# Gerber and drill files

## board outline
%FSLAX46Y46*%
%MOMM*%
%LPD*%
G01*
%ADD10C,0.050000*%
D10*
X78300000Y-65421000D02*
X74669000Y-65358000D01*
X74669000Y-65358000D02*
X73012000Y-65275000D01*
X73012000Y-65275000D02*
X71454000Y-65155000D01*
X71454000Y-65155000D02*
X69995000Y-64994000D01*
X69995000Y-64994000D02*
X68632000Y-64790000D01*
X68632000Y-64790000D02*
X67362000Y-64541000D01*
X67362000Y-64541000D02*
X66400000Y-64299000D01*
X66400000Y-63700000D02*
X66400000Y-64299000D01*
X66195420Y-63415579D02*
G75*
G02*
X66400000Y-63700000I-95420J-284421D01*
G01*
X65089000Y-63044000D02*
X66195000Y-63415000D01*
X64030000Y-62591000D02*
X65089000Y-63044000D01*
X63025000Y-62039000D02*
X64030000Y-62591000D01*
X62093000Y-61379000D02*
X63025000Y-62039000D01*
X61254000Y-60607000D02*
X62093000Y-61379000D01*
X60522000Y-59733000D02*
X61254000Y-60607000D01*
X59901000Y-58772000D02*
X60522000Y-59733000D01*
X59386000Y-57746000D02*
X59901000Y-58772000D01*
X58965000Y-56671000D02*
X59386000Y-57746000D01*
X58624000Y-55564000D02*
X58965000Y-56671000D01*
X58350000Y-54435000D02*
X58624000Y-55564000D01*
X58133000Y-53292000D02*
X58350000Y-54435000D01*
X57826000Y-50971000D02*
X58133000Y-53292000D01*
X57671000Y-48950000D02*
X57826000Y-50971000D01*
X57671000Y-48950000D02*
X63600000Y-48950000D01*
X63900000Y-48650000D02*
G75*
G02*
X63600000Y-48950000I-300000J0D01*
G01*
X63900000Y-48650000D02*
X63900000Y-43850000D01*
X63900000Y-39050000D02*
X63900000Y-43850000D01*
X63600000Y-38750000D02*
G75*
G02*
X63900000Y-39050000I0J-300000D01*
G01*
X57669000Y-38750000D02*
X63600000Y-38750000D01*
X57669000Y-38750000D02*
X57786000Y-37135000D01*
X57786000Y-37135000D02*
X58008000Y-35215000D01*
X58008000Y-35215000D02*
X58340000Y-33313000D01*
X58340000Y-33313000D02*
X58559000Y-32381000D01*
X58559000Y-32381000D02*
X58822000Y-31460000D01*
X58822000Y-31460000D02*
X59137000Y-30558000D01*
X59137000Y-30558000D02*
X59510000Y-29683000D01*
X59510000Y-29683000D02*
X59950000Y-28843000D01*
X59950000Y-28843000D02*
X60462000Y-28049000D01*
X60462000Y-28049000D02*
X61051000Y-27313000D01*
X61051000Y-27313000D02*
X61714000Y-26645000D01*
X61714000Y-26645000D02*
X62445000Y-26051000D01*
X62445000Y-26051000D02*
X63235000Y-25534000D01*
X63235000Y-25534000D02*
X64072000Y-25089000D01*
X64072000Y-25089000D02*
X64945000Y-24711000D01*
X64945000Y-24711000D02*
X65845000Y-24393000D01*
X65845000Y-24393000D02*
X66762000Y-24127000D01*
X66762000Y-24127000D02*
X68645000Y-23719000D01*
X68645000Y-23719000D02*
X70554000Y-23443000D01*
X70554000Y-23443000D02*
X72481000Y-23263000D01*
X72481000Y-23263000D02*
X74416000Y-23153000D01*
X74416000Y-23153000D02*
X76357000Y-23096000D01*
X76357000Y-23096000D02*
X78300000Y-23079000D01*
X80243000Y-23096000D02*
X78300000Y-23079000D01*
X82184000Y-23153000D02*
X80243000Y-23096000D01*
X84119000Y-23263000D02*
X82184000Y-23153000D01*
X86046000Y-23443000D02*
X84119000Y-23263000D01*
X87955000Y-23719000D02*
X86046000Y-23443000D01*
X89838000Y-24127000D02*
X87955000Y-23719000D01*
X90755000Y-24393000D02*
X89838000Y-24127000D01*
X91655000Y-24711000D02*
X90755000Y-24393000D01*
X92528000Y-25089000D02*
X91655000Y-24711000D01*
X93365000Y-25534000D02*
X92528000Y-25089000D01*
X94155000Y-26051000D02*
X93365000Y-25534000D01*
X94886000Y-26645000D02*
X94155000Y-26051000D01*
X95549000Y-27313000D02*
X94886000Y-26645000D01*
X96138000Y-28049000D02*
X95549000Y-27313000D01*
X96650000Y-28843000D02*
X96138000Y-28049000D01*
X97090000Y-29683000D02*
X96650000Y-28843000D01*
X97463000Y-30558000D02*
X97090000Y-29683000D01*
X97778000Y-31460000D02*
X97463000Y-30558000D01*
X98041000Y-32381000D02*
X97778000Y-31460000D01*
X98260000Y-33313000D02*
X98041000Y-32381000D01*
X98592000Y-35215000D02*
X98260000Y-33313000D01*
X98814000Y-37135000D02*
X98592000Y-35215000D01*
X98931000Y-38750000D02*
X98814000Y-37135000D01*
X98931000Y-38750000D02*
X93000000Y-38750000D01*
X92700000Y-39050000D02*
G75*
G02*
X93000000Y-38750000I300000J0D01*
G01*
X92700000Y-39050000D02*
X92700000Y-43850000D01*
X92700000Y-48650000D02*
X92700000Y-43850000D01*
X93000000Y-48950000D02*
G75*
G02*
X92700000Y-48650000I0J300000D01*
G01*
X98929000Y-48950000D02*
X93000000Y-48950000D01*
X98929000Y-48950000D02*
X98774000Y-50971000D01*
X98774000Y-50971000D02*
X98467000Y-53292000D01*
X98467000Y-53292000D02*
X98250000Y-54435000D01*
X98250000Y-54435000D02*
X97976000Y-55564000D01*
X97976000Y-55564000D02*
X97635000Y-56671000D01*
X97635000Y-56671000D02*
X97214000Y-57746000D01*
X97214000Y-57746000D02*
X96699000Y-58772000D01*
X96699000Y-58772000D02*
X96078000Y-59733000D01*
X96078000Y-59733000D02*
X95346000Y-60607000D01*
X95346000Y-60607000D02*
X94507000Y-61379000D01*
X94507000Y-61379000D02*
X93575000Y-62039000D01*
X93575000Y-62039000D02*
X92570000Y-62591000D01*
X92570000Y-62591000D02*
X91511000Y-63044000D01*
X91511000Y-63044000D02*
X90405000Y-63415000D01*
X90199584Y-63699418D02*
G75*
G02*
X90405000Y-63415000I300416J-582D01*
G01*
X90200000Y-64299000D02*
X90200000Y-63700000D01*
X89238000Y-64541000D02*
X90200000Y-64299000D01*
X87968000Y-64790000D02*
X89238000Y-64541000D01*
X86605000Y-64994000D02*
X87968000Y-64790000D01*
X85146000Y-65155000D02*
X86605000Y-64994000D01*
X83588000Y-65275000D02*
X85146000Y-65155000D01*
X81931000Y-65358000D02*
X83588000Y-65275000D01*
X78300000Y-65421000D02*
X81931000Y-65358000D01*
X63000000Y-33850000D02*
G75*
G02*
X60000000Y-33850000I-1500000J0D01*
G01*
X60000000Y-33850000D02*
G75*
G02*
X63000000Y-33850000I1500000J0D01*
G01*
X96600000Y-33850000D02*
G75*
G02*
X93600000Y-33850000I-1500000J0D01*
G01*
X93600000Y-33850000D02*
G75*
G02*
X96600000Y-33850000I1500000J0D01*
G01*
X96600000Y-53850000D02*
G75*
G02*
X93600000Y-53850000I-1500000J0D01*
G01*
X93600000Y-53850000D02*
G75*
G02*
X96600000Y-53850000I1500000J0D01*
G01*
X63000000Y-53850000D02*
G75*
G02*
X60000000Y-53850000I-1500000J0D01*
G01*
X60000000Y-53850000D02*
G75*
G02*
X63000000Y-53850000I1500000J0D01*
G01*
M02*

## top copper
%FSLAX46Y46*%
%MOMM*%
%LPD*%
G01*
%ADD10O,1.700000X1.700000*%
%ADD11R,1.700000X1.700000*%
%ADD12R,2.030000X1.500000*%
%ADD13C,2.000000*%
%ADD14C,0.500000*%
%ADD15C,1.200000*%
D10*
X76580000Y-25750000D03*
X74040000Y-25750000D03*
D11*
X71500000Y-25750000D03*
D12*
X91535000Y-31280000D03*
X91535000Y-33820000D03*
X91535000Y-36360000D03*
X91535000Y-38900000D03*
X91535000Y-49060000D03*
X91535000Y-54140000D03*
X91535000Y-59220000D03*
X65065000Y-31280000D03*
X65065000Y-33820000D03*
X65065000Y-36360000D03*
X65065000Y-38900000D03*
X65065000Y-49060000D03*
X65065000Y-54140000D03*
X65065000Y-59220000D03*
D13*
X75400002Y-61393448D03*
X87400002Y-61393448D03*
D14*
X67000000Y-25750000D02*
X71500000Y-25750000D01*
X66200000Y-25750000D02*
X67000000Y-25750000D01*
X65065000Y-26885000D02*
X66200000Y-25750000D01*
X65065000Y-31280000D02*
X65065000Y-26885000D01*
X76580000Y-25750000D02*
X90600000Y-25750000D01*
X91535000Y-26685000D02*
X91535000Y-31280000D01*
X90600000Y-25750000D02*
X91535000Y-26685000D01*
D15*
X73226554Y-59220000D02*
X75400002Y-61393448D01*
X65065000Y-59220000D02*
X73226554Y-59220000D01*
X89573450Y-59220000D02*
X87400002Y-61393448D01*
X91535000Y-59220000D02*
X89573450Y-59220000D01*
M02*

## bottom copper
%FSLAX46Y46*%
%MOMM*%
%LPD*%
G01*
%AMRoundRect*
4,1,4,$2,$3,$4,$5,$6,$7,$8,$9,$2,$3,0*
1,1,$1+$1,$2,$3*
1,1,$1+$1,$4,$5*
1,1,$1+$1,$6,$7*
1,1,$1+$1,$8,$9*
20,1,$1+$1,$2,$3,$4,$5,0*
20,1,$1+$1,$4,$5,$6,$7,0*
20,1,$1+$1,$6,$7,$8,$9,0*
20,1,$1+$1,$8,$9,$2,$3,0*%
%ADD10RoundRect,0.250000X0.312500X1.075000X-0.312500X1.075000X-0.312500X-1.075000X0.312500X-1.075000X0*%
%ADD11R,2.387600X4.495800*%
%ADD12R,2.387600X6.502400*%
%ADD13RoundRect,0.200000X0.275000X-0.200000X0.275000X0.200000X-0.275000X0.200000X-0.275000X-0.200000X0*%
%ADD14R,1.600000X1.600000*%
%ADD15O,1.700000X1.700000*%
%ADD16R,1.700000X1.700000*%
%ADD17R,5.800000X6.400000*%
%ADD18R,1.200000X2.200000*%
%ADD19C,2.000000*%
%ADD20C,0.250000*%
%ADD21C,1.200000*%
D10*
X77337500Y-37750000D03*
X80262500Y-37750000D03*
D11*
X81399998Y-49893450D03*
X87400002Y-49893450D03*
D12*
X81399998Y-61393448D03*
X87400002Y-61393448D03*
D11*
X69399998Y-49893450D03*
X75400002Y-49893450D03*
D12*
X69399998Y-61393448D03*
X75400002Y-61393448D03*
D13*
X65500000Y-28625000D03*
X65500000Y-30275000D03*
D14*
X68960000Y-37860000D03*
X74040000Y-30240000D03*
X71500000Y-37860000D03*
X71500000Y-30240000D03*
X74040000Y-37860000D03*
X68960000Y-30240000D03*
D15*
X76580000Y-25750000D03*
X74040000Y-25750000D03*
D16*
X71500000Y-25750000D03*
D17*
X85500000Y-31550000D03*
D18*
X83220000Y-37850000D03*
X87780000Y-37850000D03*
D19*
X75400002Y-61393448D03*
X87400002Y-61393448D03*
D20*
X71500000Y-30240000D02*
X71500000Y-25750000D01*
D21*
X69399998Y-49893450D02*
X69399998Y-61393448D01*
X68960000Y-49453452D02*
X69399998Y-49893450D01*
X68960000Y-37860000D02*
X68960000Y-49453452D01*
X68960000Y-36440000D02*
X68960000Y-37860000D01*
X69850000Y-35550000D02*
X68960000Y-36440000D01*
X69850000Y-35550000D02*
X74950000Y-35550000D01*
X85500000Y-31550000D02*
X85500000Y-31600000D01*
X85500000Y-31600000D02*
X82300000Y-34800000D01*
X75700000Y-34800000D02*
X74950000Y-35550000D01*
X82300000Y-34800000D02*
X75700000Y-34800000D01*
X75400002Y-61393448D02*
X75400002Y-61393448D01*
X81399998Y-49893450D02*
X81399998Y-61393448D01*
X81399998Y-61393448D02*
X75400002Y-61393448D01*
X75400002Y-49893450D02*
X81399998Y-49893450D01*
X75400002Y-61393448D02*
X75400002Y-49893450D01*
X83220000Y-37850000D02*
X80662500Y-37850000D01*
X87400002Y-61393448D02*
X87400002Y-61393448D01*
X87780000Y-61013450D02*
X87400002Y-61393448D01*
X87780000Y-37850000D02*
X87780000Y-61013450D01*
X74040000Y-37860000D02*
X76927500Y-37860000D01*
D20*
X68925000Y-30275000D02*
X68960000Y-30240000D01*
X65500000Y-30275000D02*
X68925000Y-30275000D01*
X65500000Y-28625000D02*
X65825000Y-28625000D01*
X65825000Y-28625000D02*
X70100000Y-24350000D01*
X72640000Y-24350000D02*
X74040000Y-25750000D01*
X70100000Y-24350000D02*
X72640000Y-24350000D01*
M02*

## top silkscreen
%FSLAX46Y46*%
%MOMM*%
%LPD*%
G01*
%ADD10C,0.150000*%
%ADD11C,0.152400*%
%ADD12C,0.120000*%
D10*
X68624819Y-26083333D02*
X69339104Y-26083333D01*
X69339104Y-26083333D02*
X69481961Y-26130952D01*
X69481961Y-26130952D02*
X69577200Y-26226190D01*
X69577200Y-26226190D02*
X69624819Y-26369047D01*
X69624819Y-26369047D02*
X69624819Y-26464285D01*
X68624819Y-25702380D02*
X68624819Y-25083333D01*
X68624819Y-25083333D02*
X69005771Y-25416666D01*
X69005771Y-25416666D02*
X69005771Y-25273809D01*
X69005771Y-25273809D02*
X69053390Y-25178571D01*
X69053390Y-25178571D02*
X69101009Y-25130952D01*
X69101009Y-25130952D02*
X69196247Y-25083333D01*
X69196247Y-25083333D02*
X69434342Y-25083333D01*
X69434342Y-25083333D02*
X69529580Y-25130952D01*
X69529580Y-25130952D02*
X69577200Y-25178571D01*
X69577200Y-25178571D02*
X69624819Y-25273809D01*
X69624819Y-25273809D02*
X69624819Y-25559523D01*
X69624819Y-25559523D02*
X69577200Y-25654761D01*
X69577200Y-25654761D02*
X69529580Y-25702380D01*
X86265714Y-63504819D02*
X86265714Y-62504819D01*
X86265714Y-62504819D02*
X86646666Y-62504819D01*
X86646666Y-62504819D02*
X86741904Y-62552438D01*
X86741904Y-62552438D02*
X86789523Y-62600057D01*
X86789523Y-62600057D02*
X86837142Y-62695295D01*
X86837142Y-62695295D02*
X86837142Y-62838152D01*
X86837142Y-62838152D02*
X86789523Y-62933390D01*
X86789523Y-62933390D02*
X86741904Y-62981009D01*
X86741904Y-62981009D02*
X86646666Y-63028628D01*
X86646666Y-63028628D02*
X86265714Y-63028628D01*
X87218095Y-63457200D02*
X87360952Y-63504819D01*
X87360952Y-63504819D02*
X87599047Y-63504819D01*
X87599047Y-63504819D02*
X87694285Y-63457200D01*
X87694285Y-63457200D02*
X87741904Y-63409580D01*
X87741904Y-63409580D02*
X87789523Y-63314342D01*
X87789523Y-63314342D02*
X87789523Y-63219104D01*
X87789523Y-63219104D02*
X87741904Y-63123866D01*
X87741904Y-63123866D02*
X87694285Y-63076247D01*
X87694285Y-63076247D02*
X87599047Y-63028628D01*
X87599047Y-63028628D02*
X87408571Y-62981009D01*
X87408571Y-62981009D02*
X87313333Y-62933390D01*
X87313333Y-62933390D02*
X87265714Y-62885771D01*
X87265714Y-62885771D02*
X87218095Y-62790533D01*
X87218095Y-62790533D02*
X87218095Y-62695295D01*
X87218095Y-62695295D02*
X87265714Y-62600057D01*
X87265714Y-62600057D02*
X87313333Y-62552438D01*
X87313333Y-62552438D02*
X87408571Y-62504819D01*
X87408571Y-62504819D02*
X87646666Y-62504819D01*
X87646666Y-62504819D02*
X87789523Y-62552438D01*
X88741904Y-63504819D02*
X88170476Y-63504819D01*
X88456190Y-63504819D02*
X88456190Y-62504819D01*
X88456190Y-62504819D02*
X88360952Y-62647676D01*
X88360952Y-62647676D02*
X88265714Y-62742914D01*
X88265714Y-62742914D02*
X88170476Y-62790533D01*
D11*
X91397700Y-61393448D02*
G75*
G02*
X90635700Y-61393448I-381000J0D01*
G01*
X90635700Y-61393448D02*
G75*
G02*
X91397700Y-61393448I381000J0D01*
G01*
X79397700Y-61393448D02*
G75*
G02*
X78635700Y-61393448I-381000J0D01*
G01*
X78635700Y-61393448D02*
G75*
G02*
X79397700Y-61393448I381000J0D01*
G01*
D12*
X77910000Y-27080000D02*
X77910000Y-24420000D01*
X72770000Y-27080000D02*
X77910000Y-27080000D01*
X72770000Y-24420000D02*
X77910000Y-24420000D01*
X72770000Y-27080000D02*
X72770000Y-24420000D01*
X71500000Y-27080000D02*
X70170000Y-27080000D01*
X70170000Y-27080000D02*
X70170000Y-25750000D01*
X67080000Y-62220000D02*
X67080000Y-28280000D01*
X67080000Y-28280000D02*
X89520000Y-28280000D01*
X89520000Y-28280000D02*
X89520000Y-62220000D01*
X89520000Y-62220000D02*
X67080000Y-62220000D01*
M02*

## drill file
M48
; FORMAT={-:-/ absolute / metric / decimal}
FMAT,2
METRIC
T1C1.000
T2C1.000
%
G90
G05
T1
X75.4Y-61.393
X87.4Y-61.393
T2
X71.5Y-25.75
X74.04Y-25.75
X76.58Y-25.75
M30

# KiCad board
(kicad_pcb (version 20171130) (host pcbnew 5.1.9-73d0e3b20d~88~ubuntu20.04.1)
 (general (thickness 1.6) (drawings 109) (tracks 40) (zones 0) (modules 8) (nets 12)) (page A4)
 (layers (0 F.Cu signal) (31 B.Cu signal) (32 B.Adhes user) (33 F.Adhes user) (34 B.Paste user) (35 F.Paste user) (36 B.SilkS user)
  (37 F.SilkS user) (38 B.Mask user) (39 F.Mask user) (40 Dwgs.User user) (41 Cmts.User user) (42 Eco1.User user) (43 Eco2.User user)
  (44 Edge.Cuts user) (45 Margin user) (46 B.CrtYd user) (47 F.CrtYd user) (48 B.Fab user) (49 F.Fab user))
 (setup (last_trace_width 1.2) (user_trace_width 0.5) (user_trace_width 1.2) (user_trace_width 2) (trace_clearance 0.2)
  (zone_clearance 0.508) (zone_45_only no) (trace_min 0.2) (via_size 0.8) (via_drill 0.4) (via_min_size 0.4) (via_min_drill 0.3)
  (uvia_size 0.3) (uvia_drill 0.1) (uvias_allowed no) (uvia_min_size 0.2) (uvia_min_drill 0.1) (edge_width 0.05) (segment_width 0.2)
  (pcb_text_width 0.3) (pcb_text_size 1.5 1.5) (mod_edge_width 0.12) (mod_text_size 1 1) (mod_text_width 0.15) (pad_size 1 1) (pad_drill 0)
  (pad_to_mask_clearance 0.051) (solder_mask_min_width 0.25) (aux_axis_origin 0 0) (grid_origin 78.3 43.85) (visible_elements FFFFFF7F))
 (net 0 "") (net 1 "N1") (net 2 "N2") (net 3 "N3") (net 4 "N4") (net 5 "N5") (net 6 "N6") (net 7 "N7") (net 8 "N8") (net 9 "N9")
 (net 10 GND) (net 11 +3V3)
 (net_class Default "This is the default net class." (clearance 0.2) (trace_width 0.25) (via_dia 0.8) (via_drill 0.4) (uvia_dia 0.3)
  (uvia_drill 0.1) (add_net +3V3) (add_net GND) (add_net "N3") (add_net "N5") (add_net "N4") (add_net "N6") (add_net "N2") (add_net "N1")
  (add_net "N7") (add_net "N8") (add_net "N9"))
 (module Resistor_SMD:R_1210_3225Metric (layer B.Cu) (at 78.8 37.75 180)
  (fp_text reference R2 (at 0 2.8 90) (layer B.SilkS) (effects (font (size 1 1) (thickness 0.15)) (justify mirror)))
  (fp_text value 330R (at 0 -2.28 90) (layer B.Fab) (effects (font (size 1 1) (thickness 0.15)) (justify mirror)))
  (pad 2 smd roundrect (at 1.4625 0 180) (size 1.125 2.65) (layers B.Cu B.Paste B.Mask) (roundrect_rratio 0.222222) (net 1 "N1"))
  (pad 1 smd roundrect (at -1.4625 0 180) (size 1.125 2.65) (layers B.Cu B.Paste B.Mask) (roundrect_rratio 0.222222) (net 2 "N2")))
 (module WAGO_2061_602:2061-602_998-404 (layer B.Cu) (at 84.4 56.65 180)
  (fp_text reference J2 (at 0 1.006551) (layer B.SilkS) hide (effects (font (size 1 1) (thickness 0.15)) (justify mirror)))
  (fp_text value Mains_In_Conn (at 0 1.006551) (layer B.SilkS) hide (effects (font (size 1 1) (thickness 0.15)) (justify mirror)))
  (fp_circle (center -6.6167 -4.743448) (end -6.2357 -4.743448) (layer F.SilkS) (width 0.1524))
  (pad 2 smd rect (at 3.000002 6.75655 180) (size 2.3876 4.4958) (layers B.Cu B.Paste B.Mask) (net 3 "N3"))
  (pad 1 smd rect (at -3.000002 6.75655 180) (size 2.3876 4.4958) (layers B.Cu B.Paste B.Mask) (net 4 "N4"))
  (pad 2 smd rect (at 3.000002 -4.743448 180) (size 2.3876 6.5024) (layers B.Cu B.Paste B.Mask) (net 3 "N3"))
  (pad 1 smd rect (at -3.000002 -4.743448 180) (size 2.3876 6.5024) (layers B.Cu B.Paste B.Mask) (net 4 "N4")))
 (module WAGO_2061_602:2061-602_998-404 (layer B.Cu) (at 72.4 56.65 180)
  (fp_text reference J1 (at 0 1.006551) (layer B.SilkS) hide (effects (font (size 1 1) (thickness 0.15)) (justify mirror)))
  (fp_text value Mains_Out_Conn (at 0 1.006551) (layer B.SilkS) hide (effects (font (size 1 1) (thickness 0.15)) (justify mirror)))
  (fp_circle (center -6.6167 -4.743448) (end -6.2357 -4.743448) (layer F.SilkS) (width 0.1524))
  (pad 2 smd rect (at 3.000002 6.75655 180) (size 2.3876 4.4958) (layers B.Cu B.Paste B.Mask) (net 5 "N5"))
  (pad 1 smd rect (at -3.000002 6.75655 180) (size 2.3876 4.4958) (layers B.Cu B.Paste B.Mask) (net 3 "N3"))
  (pad 2 smd rect (at 3.000002 -4.743448 180) (size 2.3876 6.5024) (layers B.Cu B.Paste B.Mask) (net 5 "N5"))
  (pad 1 smd rect (at -3.000002 -4.743448 180) (size 2.3876 6.5024) (layers B.Cu B.Paste B.Mask) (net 3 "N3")))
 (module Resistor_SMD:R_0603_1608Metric (layer B.Cu) (at 65.5 29.45 90)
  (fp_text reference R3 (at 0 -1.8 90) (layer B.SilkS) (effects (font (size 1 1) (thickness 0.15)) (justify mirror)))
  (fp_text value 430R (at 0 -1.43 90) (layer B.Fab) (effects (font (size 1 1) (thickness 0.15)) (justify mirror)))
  (pad 2 smd roundrect (at 0.825 0 90) (size 0.8 0.95) (layers B.Cu B.Paste B.Mask) (roundrect_rratio 0.25) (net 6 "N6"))
  (pad 1 smd roundrect (at -0.825 0 90) (size 0.8 0.95) (layers B.Cu B.Paste B.Mask) (roundrect_rratio 0.25) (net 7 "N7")))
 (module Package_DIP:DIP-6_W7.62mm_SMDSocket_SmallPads (layer B.Cu) (at 71.5 34.05 270)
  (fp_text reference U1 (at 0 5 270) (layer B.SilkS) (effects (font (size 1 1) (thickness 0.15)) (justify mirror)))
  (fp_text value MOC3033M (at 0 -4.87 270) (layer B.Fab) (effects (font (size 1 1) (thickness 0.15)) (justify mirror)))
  (pad 6 smd rect (at 3.81 2.54 270) (size 1.6 1.6) (layers B.Cu B.Paste B.Mask) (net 5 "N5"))
  (pad 3 smd rect (at -3.81 -2.54 270) (size 1.6 1.6) (layers B.Cu B.Paste B.Mask) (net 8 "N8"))
  (pad 5 smd rect (at 3.81 0 270) (size 1.6 1.6) (layers B.Cu B.Paste B.Mask) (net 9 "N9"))
  (pad 2 smd rect (at -3.81 0 270) (size 1.6 1.6) (layers B.Cu B.Paste B.Mask) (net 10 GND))
  (pad 4 smd rect (at 3.81 -2.54 270) (size 1.6 1.6) (layers B.Cu B.Paste B.Mask) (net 1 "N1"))
  (pad 1 smd rect (at -3.81 2.54 270) (size 1.6 1.6) (layers B.Cu B.Paste B.Mask) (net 7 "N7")))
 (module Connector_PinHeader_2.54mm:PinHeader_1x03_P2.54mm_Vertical (layer F.Cu) (at 71.5 25.75 90)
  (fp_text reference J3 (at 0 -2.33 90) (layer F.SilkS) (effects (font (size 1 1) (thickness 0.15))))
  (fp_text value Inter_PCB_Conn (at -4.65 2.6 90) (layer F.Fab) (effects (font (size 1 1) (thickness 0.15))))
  (fp_line (start -1.33 6.41) (end 1.33 6.41) (layer F.SilkS) (width 0.12))
  (fp_line (start -1.33 1.27) (end -1.33 6.41) (layer F.SilkS) (width 0.12))
  (fp_line (start 1.33 1.27) (end 1.33 6.41) (layer F.SilkS) (width 0.12))
  (fp_line (start -1.33 1.27) (end 1.33 1.27) (layer F.SilkS) (width 0.12))
  (fp_line (start -1.33 0) (end -1.33 -1.33) (layer F.SilkS) (width 0.12))
  (fp_line (start -1.33 -1.33) (end 0 -1.33) (layer F.SilkS) (width 0.12))
  (pad 3 thru_hole oval (at 0 5.08 90) (size 1.7 1.7) (drill 1) (layers *.Cu *.Mask) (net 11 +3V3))
  (pad 2 thru_hole oval (at 0 2.54 90) (size 1.7 1.7) (drill 1) (layers *.Cu *.Mask) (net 6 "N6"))
  (pad 1 thru_hole rect (at 0 0 90) (size 1.7 1.7) (drill 1) (layers *.Cu *.Mask) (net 10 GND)))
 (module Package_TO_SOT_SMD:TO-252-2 (layer B.Cu) (at 85.5 33.65 90)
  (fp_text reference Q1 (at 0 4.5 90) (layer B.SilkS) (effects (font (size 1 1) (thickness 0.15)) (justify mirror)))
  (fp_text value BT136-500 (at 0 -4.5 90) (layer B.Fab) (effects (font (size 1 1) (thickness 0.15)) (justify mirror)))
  (pad "" smd rect (at 0.425 -1.525 90) (size 3.05 2.75) (layers B.Paste))
  (pad "" smd rect (at 3.775 1.525 90) (size 3.05 2.75) (layers B.Paste))
  (pad "" smd rect (at 0.425 1.525 90) (size 3.05 2.75) (layers B.Paste))
  (pad "" smd rect (at 3.775 -1.525 90) (size 3.05 2.75) (layers B.Paste))
  (pad 2 smd rect (at 2.1 0 90) (size 6.4 5.8) (layers B.Cu B.Mask) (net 5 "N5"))
  (pad 3 smd rect (at -4.2 -2.28 90) (size 2.2 1.2) (layers B.Cu B.Paste B.Mask) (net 2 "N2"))
  (pad 1 smd rect (at -4.2 2.28 90) (size 2.2 1.2) (layers B.Cu B.Paste B.Mask) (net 4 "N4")))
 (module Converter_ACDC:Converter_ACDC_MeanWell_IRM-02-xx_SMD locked (layer F.Cu) (at 78.3 45.25 180)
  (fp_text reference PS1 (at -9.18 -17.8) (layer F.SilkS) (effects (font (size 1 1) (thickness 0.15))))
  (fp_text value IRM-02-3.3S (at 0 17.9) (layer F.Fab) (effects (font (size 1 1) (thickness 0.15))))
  (fp_line (start 11.22 -16.97) (end 11.22 16.97) (layer F.SilkS) (width 0.12))
  (fp_line (start 11.22 16.97) (end -11.22 16.97) (layer F.SilkS) (width 0.12))
  (fp_line (start -11.22 16.97) (end -11.22 -16.97) (layer F.SilkS) (width 0.12))
  (fp_line (start -11.22 -16.97) (end 11.22 -16.97) (layer F.SilkS) (width 0.12))
  (pad 12 smd rect (at -13.235 13.97 90) (size 1.5 2.03) (layers F.Cu F.Paste F.Mask) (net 11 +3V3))
  (pad 11 smd rect (at -13.235 11.43 90) (size 1.5 2.03) (layers F.Cu F.Paste F.Mask))
  (pad 10 smd rect (at -13.235 8.89 90) (size 1.5 2.03) (layers F.Cu F.Paste F.Mask))
  (pad 9 smd rect (at -13.235 6.35 90) (size 1.5 2.03) (layers F.Cu F.Paste F.Mask))
  (pad 5 smd rect (at -13.235 -3.81 90) (size 1.5 2.03) (layers F.Cu F.Paste F.Mask))
  (pad 3 smd rect (at -13.235 -8.89 90) (size 1.5 2.03) (layers F.Cu F.Paste F.Mask))
  (pad 1 smd rect (at -13.235 -13.97 90) (size 1.5 2.03) (layers F.Cu F.Paste F.Mask) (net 4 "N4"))
  (pad 13 smd rect (at 13.235 13.97 90) (size 1.5 2.03) (layers F.Cu F.Paste F.Mask) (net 10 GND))
  (pad 14 smd rect (at 13.235 11.43 90) (size 1.5 2.03) (layers F.Cu F.Paste F.Mask))
  (pad 15 smd rect (at 13.235 8.89 90) (size 1.5 2.03) (layers F.Cu F.Paste F.Mask))
  (pad 16 smd rect (at 13.235 6.35 90) (size 1.5 2.03) (layers F.Cu F.Paste F.Mask))
  (pad 20 smd rect (at 13.235 -3.81 90) (size 1.5 2.03) (layers F.Cu F.Paste F.Mask))
  (pad 22 smd rect (at 13.235 -8.89 90) (size 1.5 2.03) (layers F.Cu F.Paste F.Mask))
  (pad 24 smd rect (at 13.235 -13.97 90) (size 1.5 2.03) (layers F.Cu F.Paste F.Mask) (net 3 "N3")))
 (gr_line (start 78.3 65.421) (end 74.669 65.358) (angle 90) (layer Edge.Cuts) (width 0.05))
 (gr_line (start 74.669 65.358) (end 73.012 65.275) (angle 90) (layer Edge.Cuts) (width 0.05))
 (gr_line (start 73.012 65.275) (end 71.454 65.155) (angle 90) (layer Edge.Cuts) (width 0.05))
 (gr_line (start 71.454 65.155) (end 69.995 64.994) (angle 90) (layer Edge.Cuts) (width 0.05))
 (gr_line (start 69.995 64.994) (end 68.632 64.79) (angle 90) (layer Edge.Cuts) (width 0.05))
 (gr_line (start 68.632 64.79) (end 67.362 64.541) (angle 90) (layer Edge.Cuts) (width 0.05))
 (gr_line (start 67.362 64.541) (end 66.4 64.299) (angle 90) (layer Edge.Cuts) (width 0.05))
 (gr_line (start 66.4 63.7) (end 66.4 64.299) (angle 90) (layer Edge.Cuts) (width 0.05))
 (gr_arc (start 66.1 63.7) (end 66.4 63.7) (angle -71.454) (layer Edge.Cuts) (width 0.05))
 (gr_line (start 65.089 63.044) (end 66.195 63.415) (angle 90) (layer Edge.Cuts) (width 0.05))
 (gr_line (start 64.03 62.591) (end 65.089 63.044) (angle 90) (layer Edge.Cuts) (width 0.05))
 (gr_line (start 63.025 62.039) (end 64.03 62.591) (angle 90) (layer Edge.Cuts) (width 0.05))
 (gr_line (start 62.093 61.379) (end 63.025 62.039) (angle 90) (layer Edge.Cuts) (width 0.05))
 (gr_line (start 61.254 60.607) (end 62.093 61.379) (angle 90) (layer Edge.Cuts) (width 0.05))
 (gr_line (start 60.522 59.733) (end 61.254 60.607) (angle 90) (layer Edge.Cuts) (width 0.05))
 (gr_line (start 59.901 58.772) (end 60.522 59.733) (angle 90) (layer Edge.Cuts) (width 0.05))
 (gr_line (start 59.386 57.746) (end 59.901 58.772) (angle 90) (layer Edge.Cuts) (width 0.05))
 (gr_line (start 58.965 56.671) (end 59.386 57.746) (angle 90) (layer Edge.Cuts) (width 0.05))
 (gr_line (start 58.624 55.564) (end 58.965 56.671) (angle 90) (layer Edge.Cuts) (width 0.05))
 (gr_line (start 58.35 54.435) (end 58.624 55.564) (angle 90) (layer Edge.Cuts) (width 0.05))
 (gr_line (start 58.133 53.292) (end 58.35 54.435) (angle 90) (layer Edge.Cuts) (width 0.05))
 (gr_line (start 57.826 50.971) (end 58.133 53.292) (angle 90) (layer Edge.Cuts) (width 0.05))
 (gr_line (start 57.671 48.95) (end 57.826 50.971) (angle 90) (layer Edge.Cuts) (width 0.05))
 (gr_line (start 57.671 48.95) (end 63.6 48.95) (angle 90) (layer Edge.Cuts) (width 0.05))
 (gr_arc (start 63.6 48.65) (end 63.6 48.95) (angle -90) (layer Edge.Cuts) (width 0.05))
 (gr_line (start 63.9 48.65) (end 63.9 43.85) (angle 90) (layer Edge.Cuts) (width 0.05))
 (gr_line (start 63.9 39.05) (end 63.9 43.85) (angle 90) (layer Edge.Cuts) (width 0.05))
 (gr_arc (start 63.6 39.05) (end 63.9 39.05) (angle -90) (layer Edge.Cuts) (width 0.05))
 (gr_line (start 57.669 38.75) (end 63.6 38.75) (angle 90) (layer Edge.Cuts) (width 0.05))
 (gr_line (start 57.669 38.75) (end 57.786 37.135) (angle 90) (layer Edge.Cuts) (width 0.05))
 (gr_line (start 57.786 37.135) (end 58.008 35.215) (angle 90) (layer Edge.Cuts) (width 0.05))
 (gr_line (start 58.008 35.215) (end 58.34 33.313) (angle 90) (layer Edge.Cuts) (width 0.05))
 (gr_line (start 58.34 33.313) (end 58.559 32.381) (angle 90) (layer Edge.Cuts) (width 0.05))
 (gr_line (start 58.559 32.381) (end 58.822 31.46) (angle 90) (layer Edge.Cuts) (width 0.05))
 (gr_line (start 58.822 31.46) (end 59.137 30.558) (angle 90) (layer Edge.Cuts) (width 0.05))
 (gr_line (start 59.137 30.558) (end 59.51 29.683) (angle 90) (layer Edge.Cuts) (width 0.05))
 (gr_line (start 59.51 29.683) (end 59.95 28.843) (angle 90) (layer Edge.Cuts) (width 0.05))
 (gr_line (start 59.95 28.843) (end 60.462 28.049) (angle 90) (layer Edge.Cuts) (width 0.05))
 (gr_line (start 60.462 28.049) (end 61.051 27.313) (angle 90) (layer Edge.Cuts) (width 0.05))
 (gr_line (start 61.051 27.313) (end 61.714 26.645) (angle 90) (layer Edge.Cuts) (width 0.05))
 (gr_line (start 61.714 26.645) (end 62.445 26.051) (angle 90) (layer Edge.Cuts) (width 0.05))
 (gr_line (start 62.445 26.051) (end 63.235 25.534) (angle 90) (layer Edge.Cuts) (width 0.05))
 (gr_line (start 63.235 25.534) (end 64.072 25.089) (angle 90) (layer Edge.Cuts) (width 0.05))
 (gr_line (start 64.072 25.089) (end 64.945 24.711) (angle 90) (layer Edge.Cuts) (width 0.05))
 (gr_line (start 64.945 24.711) (end 65.845 24.393) (angle 90) (layer Edge.Cuts) (width 0.05))
 (gr_line (start 65.845 24.393) (end 66.762 24.127) (angle 90) (layer Edge.Cuts) (width 0.05))
 (gr_line (start 66.762 24.127) (end 68.645 23.719) (angle 90) (layer Edge.Cuts) (width 0.05))
 (gr_line (start 68.645 23.719) (end 70.554 23.443) (angle 90) (layer Edge.Cuts) (width 0.05))
 (gr_line (start 70.554 23.443) (end 72.481 23.263) (angle 90) (layer Edge.Cuts) (width 0.05))
 (gr_line (start 72.481 23.263) (end 74.416 23.153) (angle 90) (layer Edge.Cuts) (width 0.05))
 (gr_line (start 74.416 23.153) (end 76.357 23.096) (angle 90) (layer Edge.Cuts) (width 0.05))
 (gr_line (start 76.357 23.096) (end 78.3 23.079) (angle 90) (layer Edge.Cuts) (width 0.05))
 (gr_line (start 80.243 23.096) (end 78.3 23.079) (angle 90) (layer Edge.Cuts) (width 0.05))
 (gr_line (start 82.184 23.153) (end 80.243 23.096) (angle 90) (layer Edge.Cuts) (width 0.05))
 (gr_line (start 84.119 23.263) (end 82.184 23.153) (angle 90) (layer Edge.Cuts) (width 0.05))
 (gr_line (start 86.046 23.443) (end 84.119 23.263) (angle 90) (layer Edge.Cuts) (width 0.05))
 (gr_line (start 87.955 23.719) (end 86.046 23.443) (angle 90) (layer Edge.Cuts) (width 0.05))
 (gr_line (start 89.838 24.127) (end 87.955 23.719) (angle 90) (layer Edge.Cuts) (width 0.05))
 (gr_line (start 90.755 24.393) (end 89.838 24.127) (angle 90) (layer Edge.Cuts) (width 0.05))
 (gr_line (start 91.655 24.711) (end 90.755 24.393) (angle 90) (layer Edge.Cuts) (width 0.05))
 (gr_line (start 92.528 25.089) (end 91.655 24.711) (angle 90) (layer Edge.Cuts) (width 0.05))
 (gr_line (start 93.365 25.534) (end 92.528 25.089) (angle 90) (layer Edge.Cuts) (width 0.05))
 (gr_line (start 94.155 26.051) (end 93.365 25.534) (angle 90) (layer Edge.Cuts) (width 0.05))
 (gr_line (start 94.886 26.645) (end 94.155 26.051) (angle 90) (layer Edge.Cuts) (width 0.05))
 (gr_line (start 95.549 27.313) (end 94.886 26.645) (angle 90) (layer Edge.Cuts) (width 0.05))
 (gr_line (start 96.138 28.049) (end 95.549 27.313) (angle 90) (layer Edge.Cuts) (width 0.05))
 (gr_line (start 96.65 28.843) (end 96.138 28.049) (angle 90) (layer Edge.Cuts) (width 0.05))
 (gr_line (start 97.09 29.683) (end 96.65 28.843) (angle 90) (layer Edge.Cuts) (width 0.05))
 (gr_line (start 97.463 30.558) (end 97.09 29.683) (angle 90) (layer Edge.Cuts) (width 0.05))
 (gr_line (start 97.778 31.46) (end 97.463 30.558) (angle 90) (layer Edge.Cuts) (width 0.05))
 (gr_line (start 98.041 32.381) (end 97.778 31.46) (angle 90) (layer Edge.Cuts) (width 0.05))
 (gr_line (start 98.26 33.313) (end 98.041 32.381) (angle 90) (layer Edge.Cuts) (width 0.05))
 (gr_line (start 98.592 35.215) (end 98.26 33.313) (angle 90) (layer Edge.Cuts) (width 0.05))
 (gr_line (start 98.814 37.135) (end 98.592 35.215) (angle 90) (layer Edge.Cuts) (width 0.05))
 (gr_line (start 98.931 38.75) (end 98.814 37.135) (angle 90) (layer Edge.Cuts) (width 0.05))
 (gr_line (start 98.931 38.75) (end 93 38.75) (angle 90) (layer Edge.Cuts) (width 0.05))
 (gr_arc (start 93 39.05) (end 93 38.75) (angle -90) (layer Edge.Cuts) (width 0.05))
 (gr_line (start 92.7 39.05) (end 92.7 43.85) (angle 90) (layer Edge.Cuts) (width 0.05))
 (gr_line (start 92.7 48.65) (end 92.7 43.85) (angle 90) (layer Edge.Cuts) (width 0.05))
 (gr_arc (start 93 48.65) (end 92.7 48.65) (angle -90) (layer Edge.Cuts) (width 0.05))
 (gr_line (start 98.929 48.95) (end 93 48.95) (angle 90) (layer Edge.Cuts) (width 0.05))
 (gr_line (start 98.929 48.95) (end 98.774 50.971) (angle 90) (layer Edge.Cuts) (width 0.05))
 (gr_line (start 98.774 50.971) (end 98.467 53.292) (angle 90) (layer Edge.Cuts) (width 0.05))
 (gr_line (start 98.467 53.292) (end 98.25 54.435) (angle 90) (layer Edge.Cuts) (width 0.05))
 (gr_line (start 98.25 54.435) (end 97.976 55.564) (angle 90) (layer Edge.Cuts) (width 0.05))
 (gr_line (start 97.976 55.564) (end 97.635 56.671) (angle 90) (layer Edge.Cuts) (width 0.05))
 (gr_line (start 97.635 56.671) (end 97.214 57.746) (angle 90) (layer Edge.Cuts) (width 0.05))
 (gr_line (start 97.214 57.746) (end 96.699 58.772) (angle 90) (layer Edge.Cuts) (width 0.05))
 (gr_line (start 96.699 58.772) (end 96.078 59.733) (angle 90) (layer Edge.Cuts) (width 0.05))
 (gr_line (start 96.078 59.733) (end 95.346 60.607) (angle 90) (layer Edge.Cuts) (width 0.05))
 (gr_line (start 95.346 60.607) (end 94.507 61.379) (angle 90) (layer Edge.Cuts) (width 0.05))
 (gr_line (start 94.507 61.379) (end 93.575 62.039) (angle 90) (layer Edge.Cuts) (width 0.05))
 (gr_line (start 93.575 62.039) (end 92.57 62.591) (angle 90) (layer Edge.Cuts) (width 0.05))
 (gr_line (start 92.57 62.591) (end 91.511 63.044) (angle 90) (layer Edge.Cuts) (width 0.05))
 (gr_line (start 91.511 63.044) (end 90.405 63.415) (angle 90) (layer Edge.Cuts) (width 0.05))
 (gr_arc (start 90.5 63.7) (end 90.405 63.415) (angle -71.454) (layer Edge.Cuts) (width 0.05))
 (gr_line (start 90.2 64.299) (end 90.2 63.7) (angle 90) (layer Edge.Cuts) (width 0.05))
 (gr_line (start 89.238 64.541) (end 90.2 64.299) (angle 90) (layer Edge.Cuts) (width 0.05))
 (gr_line (start 87.968 64.79) (end 89.238 64.541) (angle 90) (layer Edge.Cuts) (width 0.05))
 (gr_line (start 86.605 64.994) (end 87.968 64.79) (angle 90) (layer Edge.Cuts) (width 0.05))
 (gr_line (start 85.146 65.155) (end 86.605 64.994) (angle 90) (layer Edge.Cuts) (width 0.05))
 (gr_line (start 83.588 65.275) (end 85.146 65.155) (angle 90) (layer Edge.Cuts) (width 0.05))
 (gr_line (start 81.931 65.358) (end 83.588 65.275) (angle 90) (layer Edge.Cuts) (width 0.05))
 (gr_line (start 78.3 65.421) (end 81.931 65.358) (angle 90) (layer Edge.Cuts) (width 0.05))
 (gr_circle (center 61.5 33.85) (end 60 33.85) (layer Edge.Cuts) (width 0.05))
 (gr_circle (center 95.1 33.85) (end 93.6 33.85) (layer Edge.Cuts) (width 0.05))
 (gr_circle (center 95.1 53.85) (end 93.6 53.85) (layer Edge.Cuts) (width 0.05))
 (gr_circle (center 61.5 53.85) (end 60 53.85) (layer Edge.Cuts) (width 0.05))
 (segment (start 71.5 30.24) (end 71.5 25.75) (width 0.25) (layer B.Cu) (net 10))
 (segment (start 67 25.75) (end 71.5 25.75) (width 0.5) (layer F.Cu) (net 10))
 (segment (start 66.2 25.75) (end 67 25.75) (width 0.5) (layer F.Cu) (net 10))
 (segment (start 65.065 26.885) (end 66.2 25.75) (width 0.5) (layer F.Cu) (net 10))
 (segment (start 65.065 31.28) (end 65.065 26.885) (width 0.5) (layer F.Cu) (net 10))
 (segment (start 76.58 25.75) (end 90.6 25.75) (width 0.5) (layer F.Cu) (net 11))
 (segment (start 91.535 26.685) (end 91.535 31.28) (width 0.5) (layer F.Cu) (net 11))
 (segment (start 90.6 25.75) (end 91.535 26.685) (width 0.5) (layer F.Cu) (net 11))
 (segment (start 69.399998 49.89345) (end 69.399998 61.393448) (width 1.2) (layer B.Cu) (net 5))
 (segment (start 68.96 49.453452) (end 69.399998 49.89345) (width 1.2) (layer B.Cu) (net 5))
 (segment (start 68.96 37.86) (end 68.96 49.453452) (width 1.2) (layer B.Cu) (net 5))
 (segment (start 68.96 36.44) (end 68.96 37.86) (width 1.2) (layer B.Cu) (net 5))
 (segment (start 69.85 35.55) (end 68.96 36.44) (width 1.2) (layer B.Cu) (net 5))
 (segment (start 69.85 35.55) (end 74.95 35.55) (width 1.2) (layer B.Cu) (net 5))
 (segment (start 85.5 31.55) (end 85.5 31.6) (width 1.2) (layer B.Cu) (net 5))
 (segment (start 85.5 31.6) (end 82.3 34.8) (width 1.2) (layer B.Cu) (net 5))
 (segment (start 75.7 34.8) (end 74.95 35.55) (width 1.2) (layer B.Cu) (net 5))
 (segment (start 82.3 34.8) (end 75.7 34.8) (width 1.2) (layer B.Cu) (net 5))
 (segment (start 75.400002 61.393448) (end 75.400002 61.393448) (width 1.2) (layer B.Cu) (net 3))
 (segment (start 81.399998 49.89345) (end 81.399998 61.393448) (width 1.2) (layer B.Cu) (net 3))
 (segment (start 81.399998 61.393448) (end 75.400002 61.393448) (width 1.2) (layer B.Cu) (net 3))
 (segment (start 75.400002 49.89345) (end 81.399998 49.89345) (width 1.2) (layer B.Cu) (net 3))
 (segment (start 75.400002 61.393448) (end 75.400002 49.89345) (width 1.2) (layer B.Cu) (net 3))
 (via (at 75.400002 61.393448) (size 2) (drill 1) (layers F.Cu B.Cu) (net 3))
 (segment (start 73.226554 59.22) (end 75.400002 61.393448) (width 1.2) (layer F.Cu) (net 3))
 (segment (start 65.065 59.22) (end 73.226554 59.22) (width 1.2) (layer F.Cu) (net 3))
 (segment (start 83.22 37.85) (end 80.6625 37.85) (width 1.2) (layer B.Cu) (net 2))
 (segment (start 87.400002 61.393448) (end 87.400002 61.393448) (width 1.2) (layer B.Cu) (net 4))
 (via (at 87.400002 61.393448) (size 2) (drill 1) (layers F.Cu B.Cu) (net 4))
 (segment (start 89.57345 59.22) (end 87.400002 61.393448) (width 1.2) (layer F.Cu) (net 4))
 (segment (start 91.535 59.22) (end 89.57345 59.22) (width 1.2) (layer F.Cu) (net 4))
 (segment (start 87.78 61.01345) (end 87.400002 61.393448) (width 1.2) (layer B.Cu) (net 4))
 (segment (start 87.78 37.85) (end 87.78 61.01345) (width 1.2) (layer B.Cu) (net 4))
 (segment (start 74.04 37.86) (end 76.9275 37.86) (width 1.2) (layer B.Cu) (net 1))
 (segment (start 68.925 30.275) (end 68.96 30.24) (width 0.25) (layer B.Cu) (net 7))
 (segment (start 65.5 30.275) (end 68.925 30.275) (width 0.25) (layer B.Cu) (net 7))
 (segment (start 65.5 28.625) (end 65.825 28.625) (width 0.25) (layer B.Cu) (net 6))
 (segment (start 65.825 28.625) (end 70.1 24.35) (width 0.25) (layer B.Cu) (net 6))
 (segment (start 72.64 24.35) (end 74.04 25.75) (width 0.25) (layer B.Cu) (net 6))
 (segment (start 70.1 24.35) (end 72.64 24.35) (width 0.25) (layer B.Cu) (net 6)))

